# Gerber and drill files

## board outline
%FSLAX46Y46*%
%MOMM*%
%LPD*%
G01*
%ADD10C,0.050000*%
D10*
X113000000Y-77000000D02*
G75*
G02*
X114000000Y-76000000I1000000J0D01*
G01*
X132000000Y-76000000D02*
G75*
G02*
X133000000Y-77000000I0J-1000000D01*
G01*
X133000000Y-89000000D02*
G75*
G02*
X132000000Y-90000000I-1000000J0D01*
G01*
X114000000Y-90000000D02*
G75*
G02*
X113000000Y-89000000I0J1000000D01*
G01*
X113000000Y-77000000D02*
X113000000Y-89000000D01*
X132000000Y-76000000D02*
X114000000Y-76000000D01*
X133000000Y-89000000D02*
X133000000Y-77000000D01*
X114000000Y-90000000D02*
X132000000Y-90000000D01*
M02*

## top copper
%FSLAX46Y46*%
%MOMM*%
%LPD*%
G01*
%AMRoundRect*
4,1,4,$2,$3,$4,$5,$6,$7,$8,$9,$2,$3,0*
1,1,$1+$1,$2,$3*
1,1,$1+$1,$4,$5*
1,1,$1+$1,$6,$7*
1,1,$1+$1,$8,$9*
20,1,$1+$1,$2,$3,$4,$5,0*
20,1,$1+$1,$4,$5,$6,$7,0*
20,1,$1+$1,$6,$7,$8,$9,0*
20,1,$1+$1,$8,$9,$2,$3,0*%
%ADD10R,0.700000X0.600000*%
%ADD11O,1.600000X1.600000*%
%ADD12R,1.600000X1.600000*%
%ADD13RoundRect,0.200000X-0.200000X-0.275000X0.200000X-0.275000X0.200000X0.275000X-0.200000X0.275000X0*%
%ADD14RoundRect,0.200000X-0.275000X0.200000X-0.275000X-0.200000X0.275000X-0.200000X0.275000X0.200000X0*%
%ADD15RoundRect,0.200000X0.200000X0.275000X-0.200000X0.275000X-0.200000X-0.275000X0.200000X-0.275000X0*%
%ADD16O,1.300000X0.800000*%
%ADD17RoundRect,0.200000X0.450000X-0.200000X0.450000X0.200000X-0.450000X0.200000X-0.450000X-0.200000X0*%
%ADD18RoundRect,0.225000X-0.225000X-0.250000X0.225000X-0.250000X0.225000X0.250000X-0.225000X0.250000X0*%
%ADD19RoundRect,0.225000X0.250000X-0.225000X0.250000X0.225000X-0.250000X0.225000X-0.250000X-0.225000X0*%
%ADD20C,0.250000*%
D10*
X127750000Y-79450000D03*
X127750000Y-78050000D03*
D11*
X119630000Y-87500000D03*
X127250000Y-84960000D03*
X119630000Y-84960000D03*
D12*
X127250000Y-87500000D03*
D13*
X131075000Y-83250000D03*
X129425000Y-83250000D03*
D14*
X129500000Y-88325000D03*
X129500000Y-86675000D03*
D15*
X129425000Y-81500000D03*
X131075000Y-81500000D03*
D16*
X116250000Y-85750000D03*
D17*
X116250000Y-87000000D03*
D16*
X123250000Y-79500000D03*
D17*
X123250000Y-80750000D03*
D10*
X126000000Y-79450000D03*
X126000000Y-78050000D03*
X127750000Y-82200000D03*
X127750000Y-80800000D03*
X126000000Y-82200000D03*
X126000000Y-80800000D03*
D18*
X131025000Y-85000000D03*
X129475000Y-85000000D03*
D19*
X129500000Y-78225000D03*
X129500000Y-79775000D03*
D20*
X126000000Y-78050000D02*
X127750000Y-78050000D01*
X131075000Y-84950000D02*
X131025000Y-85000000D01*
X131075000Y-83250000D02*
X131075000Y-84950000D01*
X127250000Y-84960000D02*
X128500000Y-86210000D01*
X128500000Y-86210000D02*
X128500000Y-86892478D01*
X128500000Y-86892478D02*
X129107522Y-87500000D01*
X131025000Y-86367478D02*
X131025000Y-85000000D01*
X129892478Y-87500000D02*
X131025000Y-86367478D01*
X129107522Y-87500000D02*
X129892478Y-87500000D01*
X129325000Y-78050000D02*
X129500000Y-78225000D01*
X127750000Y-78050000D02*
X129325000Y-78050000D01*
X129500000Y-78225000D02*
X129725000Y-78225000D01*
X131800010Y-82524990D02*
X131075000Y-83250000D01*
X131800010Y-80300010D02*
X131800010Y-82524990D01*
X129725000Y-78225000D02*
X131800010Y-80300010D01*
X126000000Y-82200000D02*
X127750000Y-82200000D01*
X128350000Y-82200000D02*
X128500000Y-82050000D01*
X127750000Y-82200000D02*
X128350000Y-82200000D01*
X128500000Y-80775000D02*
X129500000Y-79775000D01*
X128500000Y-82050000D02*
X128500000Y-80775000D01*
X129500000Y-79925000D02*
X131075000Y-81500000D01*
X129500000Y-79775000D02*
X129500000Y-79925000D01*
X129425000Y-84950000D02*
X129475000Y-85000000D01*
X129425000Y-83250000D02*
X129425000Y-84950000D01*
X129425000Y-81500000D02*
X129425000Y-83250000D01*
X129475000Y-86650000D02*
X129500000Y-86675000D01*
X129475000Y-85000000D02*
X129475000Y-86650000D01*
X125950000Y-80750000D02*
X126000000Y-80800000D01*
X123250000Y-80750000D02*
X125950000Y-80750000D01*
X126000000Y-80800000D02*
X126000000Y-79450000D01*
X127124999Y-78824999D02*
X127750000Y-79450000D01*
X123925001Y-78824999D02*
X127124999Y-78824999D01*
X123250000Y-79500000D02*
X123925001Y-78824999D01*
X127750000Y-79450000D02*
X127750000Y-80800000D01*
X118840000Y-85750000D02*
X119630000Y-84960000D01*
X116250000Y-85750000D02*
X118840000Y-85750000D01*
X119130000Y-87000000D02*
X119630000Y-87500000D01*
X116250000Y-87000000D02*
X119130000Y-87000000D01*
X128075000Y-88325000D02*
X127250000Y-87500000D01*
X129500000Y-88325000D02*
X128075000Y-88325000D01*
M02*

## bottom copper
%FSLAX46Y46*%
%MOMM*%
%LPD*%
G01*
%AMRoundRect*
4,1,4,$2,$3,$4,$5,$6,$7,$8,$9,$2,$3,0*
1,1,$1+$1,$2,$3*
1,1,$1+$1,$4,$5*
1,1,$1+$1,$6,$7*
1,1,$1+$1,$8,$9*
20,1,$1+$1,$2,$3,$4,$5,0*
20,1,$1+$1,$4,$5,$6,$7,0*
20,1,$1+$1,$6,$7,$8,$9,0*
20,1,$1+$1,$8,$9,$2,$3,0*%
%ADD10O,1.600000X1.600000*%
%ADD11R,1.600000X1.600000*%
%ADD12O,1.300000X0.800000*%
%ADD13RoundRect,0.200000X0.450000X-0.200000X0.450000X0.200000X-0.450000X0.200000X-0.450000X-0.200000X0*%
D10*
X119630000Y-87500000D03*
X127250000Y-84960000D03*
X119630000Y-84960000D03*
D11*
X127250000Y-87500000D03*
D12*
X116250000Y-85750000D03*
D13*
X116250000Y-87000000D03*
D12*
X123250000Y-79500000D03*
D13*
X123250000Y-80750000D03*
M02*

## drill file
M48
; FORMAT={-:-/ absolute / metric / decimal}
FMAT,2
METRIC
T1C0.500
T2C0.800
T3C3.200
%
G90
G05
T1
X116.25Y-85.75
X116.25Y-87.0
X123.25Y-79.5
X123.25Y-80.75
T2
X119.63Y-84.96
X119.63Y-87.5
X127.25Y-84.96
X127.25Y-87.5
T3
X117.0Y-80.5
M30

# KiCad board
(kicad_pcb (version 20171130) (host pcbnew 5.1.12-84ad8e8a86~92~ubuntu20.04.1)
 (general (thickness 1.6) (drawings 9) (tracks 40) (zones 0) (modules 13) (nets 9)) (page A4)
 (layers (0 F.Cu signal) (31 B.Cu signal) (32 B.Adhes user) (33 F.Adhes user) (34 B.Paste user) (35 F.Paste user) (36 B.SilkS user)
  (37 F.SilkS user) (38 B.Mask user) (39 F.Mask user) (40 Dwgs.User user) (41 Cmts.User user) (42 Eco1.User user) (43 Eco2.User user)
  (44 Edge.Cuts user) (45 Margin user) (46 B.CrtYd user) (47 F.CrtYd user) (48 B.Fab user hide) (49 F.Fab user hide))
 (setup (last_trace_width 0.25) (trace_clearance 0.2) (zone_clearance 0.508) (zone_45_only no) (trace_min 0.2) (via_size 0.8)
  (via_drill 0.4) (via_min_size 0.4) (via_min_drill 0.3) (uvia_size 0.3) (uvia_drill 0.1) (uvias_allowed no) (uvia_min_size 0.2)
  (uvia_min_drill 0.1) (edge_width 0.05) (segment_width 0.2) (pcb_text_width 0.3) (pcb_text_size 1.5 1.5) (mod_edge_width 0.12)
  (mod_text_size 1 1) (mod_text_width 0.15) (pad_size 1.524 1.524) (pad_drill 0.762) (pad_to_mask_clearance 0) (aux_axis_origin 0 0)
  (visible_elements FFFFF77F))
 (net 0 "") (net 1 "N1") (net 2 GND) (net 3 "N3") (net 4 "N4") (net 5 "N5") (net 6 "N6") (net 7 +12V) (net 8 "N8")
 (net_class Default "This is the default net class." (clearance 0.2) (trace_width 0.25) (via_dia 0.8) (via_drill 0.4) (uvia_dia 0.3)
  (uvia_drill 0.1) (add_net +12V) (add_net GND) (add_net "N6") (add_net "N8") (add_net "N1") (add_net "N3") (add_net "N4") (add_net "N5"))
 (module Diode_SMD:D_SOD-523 (layer F.Cu) (at 127.75 78.75 90)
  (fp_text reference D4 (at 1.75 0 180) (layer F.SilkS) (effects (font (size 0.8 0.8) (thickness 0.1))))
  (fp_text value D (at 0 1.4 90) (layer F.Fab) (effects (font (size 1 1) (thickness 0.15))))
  (pad 1 smd rect (at -0.7 0 270) (size 0.6 0.7) (layers F.Cu F.Paste F.Mask) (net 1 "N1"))
  (pad 2 smd rect (at 0.7 0 270) (size 0.6 0.7) (layers F.Cu F.Paste F.Mask) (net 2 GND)))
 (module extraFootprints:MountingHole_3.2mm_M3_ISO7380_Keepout (layer F.Cu) (at 117 80.5)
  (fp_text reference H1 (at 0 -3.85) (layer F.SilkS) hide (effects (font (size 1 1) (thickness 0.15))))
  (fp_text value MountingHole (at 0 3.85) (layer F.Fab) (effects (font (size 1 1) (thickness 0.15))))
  (pad "" np_thru_hole circle (at 0 0) (size 3.2 3.2) (drill 3.2) (layers *.Cu *.Mask) (solder_mask_margin 1.45) (clearance 1.45)))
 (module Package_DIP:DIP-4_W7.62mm (layer F.Cu) (at 127.25 87.5 180)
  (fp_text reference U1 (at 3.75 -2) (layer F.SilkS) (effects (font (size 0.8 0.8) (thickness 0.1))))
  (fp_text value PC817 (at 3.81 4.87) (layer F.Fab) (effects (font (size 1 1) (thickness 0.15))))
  (pad 4 thru_hole oval (at 7.62 0 180) (size 1.6 1.6) (drill 0.8) (layers *.Cu *.Mask) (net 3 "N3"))
  (pad 2 thru_hole oval (at 0 2.54 180) (size 1.6 1.6) (drill 0.8) (layers *.Cu *.Mask) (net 2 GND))
  (pad 3 thru_hole oval (at 7.62 2.54 180) (size 1.6 1.6) (drill 0.8) (layers *.Cu *.Mask) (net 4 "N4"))
  (pad 1 thru_hole rect (at 0 0 180) (size 1.6 1.6) (drill 0.8) (layers *.Cu *.Mask) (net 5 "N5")))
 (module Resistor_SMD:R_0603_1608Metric (layer F.Cu) (at 130.25 83.25)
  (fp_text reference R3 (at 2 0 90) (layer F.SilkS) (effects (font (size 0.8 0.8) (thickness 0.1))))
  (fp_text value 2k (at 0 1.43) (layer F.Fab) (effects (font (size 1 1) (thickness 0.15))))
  (pad 2 smd roundrect (at 0.825 0) (size 0.8 0.95) (layers F.Cu F.Paste F.Mask) (roundrect_rratio 0.25) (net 2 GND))
  (pad 1 smd roundrect (at -0.825 0) (size 0.8 0.95) (layers F.Cu F.Paste F.Mask) (roundrect_rratio 0.25) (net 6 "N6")))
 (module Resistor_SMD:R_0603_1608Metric (layer F.Cu) (at 129.5 87.5 270)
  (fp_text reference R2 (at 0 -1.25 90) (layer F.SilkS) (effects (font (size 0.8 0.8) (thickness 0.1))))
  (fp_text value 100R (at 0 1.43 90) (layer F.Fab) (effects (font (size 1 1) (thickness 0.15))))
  (pad 2 smd roundrect (at 0.825 0 270) (size 0.8 0.95) (layers F.Cu F.Paste F.Mask) (roundrect_rratio 0.25) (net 5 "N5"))
  (pad 1 smd roundrect (at -0.825 0 270) (size 0.8 0.95) (layers F.Cu F.Paste F.Mask) (roundrect_rratio 0.25) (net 6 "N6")))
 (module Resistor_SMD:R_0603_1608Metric (layer F.Cu) (at 130.25 81.5 180)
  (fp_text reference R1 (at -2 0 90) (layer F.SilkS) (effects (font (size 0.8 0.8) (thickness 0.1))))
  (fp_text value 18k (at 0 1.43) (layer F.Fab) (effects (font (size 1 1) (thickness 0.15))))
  (pad 2 smd roundrect (at 0.825 0 180) (size 0.8 0.95) (layers F.Cu F.Paste F.Mask) (roundrect_rratio 0.25) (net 6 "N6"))
  (pad 1 smd roundrect (at -0.825 0 180) (size 0.8 0.95) (layers F.Cu F.Paste F.Mask) (roundrect_rratio 0.25) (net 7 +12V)))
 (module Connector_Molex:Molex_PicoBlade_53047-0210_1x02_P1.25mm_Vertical (layer F.Cu) (at 116.25 87 90)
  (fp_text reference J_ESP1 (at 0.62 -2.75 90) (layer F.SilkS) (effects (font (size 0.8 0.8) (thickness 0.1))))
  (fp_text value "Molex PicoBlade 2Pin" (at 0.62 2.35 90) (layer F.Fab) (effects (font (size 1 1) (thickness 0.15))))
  (pad 2 thru_hole oval (at 1.25 0 90) (size 0.8 1.3) (drill 0.5) (layers *.Cu *.Mask) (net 4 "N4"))
  (pad 1 thru_hole roundrect (at 0 0 90) (size 0.8 1.3) (drill 0.5) (layers *.Cu *.Mask) (roundrect_rratio 0.25) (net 3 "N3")))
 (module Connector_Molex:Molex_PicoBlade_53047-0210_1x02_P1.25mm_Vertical (layer F.Cu) (at 123.25 80.75 90)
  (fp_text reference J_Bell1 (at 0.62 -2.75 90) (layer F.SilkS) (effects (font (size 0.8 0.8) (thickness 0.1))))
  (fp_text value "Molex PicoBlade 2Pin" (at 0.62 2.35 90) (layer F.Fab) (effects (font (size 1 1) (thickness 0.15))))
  (pad 2 thru_hole oval (at 1.25 0 90) (size 0.8 1.3) (drill 0.5) (layers *.Cu *.Mask) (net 1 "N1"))
  (pad 1 thru_hole roundrect (at 0 0 90) (size 0.8 1.3) (drill 0.5) (layers *.Cu *.Mask) (roundrect_rratio 0.25) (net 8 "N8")))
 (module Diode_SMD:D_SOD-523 (layer F.Cu) (at 126 78.75 90)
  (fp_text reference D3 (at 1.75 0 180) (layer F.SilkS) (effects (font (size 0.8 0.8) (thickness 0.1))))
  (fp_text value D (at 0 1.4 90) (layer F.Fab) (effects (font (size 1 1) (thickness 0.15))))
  (pad 1 smd rect (at -0.7 0 270) (size 0.6 0.7) (layers F.Cu F.Paste F.Mask) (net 8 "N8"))
  (pad 2 smd rect (at 0.7 0 270) (size 0.6 0.7) (layers F.Cu F.Paste F.Mask) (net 2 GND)))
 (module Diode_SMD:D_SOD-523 (layer F.Cu) (at 127.75 81.5 90)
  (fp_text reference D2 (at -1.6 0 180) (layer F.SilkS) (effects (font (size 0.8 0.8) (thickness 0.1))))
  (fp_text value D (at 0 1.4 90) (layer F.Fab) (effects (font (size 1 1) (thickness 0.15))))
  (pad 1 smd rect (at -0.7 0 270) (size 0.6 0.7) (layers F.Cu F.Paste F.Mask) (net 7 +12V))
  (pad 2 smd rect (at 0.7 0 270) (size 0.6 0.7) (layers F.Cu F.Paste F.Mask) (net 1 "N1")))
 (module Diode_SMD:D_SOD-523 (layer F.Cu) (at 126 81.5 90)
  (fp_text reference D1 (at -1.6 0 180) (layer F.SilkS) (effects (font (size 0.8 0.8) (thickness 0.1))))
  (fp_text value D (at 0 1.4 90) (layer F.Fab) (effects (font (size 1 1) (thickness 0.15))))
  (pad 1 smd rect (at -0.7 0 270) (size 0.6 0.7) (layers F.Cu F.Paste F.Mask) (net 7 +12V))
  (pad 2 smd rect (at 0.7 0 270) (size 0.6 0.7) (layers F.Cu F.Paste F.Mask) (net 8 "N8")))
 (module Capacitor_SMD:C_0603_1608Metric (layer F.Cu) (at 130.25 85)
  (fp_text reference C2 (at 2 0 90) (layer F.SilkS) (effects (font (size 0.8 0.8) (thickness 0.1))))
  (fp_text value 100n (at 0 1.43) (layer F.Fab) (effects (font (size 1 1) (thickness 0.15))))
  (pad 2 smd roundrect (at 0.775 0) (size 0.9 0.95) (layers F.Cu F.Paste F.Mask) (roundrect_rratio 0.25) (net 2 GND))
  (pad 1 smd roundrect (at -0.775 0) (size 0.9 0.95) (layers F.Cu F.Paste F.Mask) (roundrect_rratio 0.25) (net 6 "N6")))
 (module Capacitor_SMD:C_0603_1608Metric (layer F.Cu) (at 129.5 79 90)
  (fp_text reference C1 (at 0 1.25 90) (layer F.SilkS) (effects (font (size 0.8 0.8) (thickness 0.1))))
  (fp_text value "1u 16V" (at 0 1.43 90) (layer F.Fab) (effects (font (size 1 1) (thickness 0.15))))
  (pad 2 smd roundrect (at 0.775 0 90) (size 0.9 0.95) (layers F.Cu F.Paste F.Mask) (roundrect_rratio 0.25) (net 2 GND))
  (pad 1 smd roundrect (at -0.775 0 90) (size 0.9 0.95) (layers F.Cu F.Paste F.Mask) (roundrect_rratio 0.25) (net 7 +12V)))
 (gr_arc (start 114 77) (end 114 76) (angle -90) (layer Edge.Cuts) (width 0.05))
 (gr_arc (start 132 77) (end 133 77) (angle -90) (layer Edge.Cuts) (width 0.05))
 (gr_arc (start 132 89) (end 132 90) (angle -90) (layer Edge.Cuts) (width 0.05))
 (gr_arc (start 114 89) (end 113 89) (angle -90) (layer Edge.Cuts) (width 0.05))
 (gr_line (start 113 77) (end 113 89) (layer Edge.Cuts) (width 0.05))
 (gr_line (start 132 76) (end 114 76) (layer Edge.Cuts) (width 0.05))
 (gr_line (start 133 89) (end 133 77) (layer Edge.Cuts) (width 0.05))
 (gr_line (start 114 90) (end 132 90) (layer Edge.Cuts) (width 0.05))
 (segment (start 126 78.05) (end 127.75 78.05) (width 0.25) (layer F.Cu) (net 2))
 (segment (start 131.075 84.95) (end 131.025 85) (width 0.25) (layer F.Cu) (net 2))
 (segment (start 131.075 83.25) (end 131.075 84.95) (width 0.25) (layer F.Cu) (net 2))
 (segment (start 127.25 84.96) (end 128.5 86.21) (width 0.25) (layer F.Cu) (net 2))
 (segment (start 128.5 86.21) (end 128.5 86.892478) (width 0.25) (layer F.Cu) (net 2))
 (segment (start 128.5 86.892478) (end 129.107522 87.5) (width 0.25) (layer F.Cu) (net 2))
 (segment (start 131.025 86.367478) (end 131.025 85) (width 0.25) (layer F.Cu) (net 2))
 (segment (start 129.892478 87.5) (end 131.025 86.367478) (width 0.25) (layer F.Cu) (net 2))
 (segment (start 129.107522 87.5) (end 129.892478 87.5) (width 0.25) (layer F.Cu) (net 2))
 (segment (start 129.325 78.05) (end 129.5 78.225) (width 0.25) (layer F.Cu) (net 2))
 (segment (start 127.75 78.05) (end 129.325 78.05) (width 0.25) (layer F.Cu) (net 2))
 (segment (start 129.5 78.225) (end 129.725 78.225) (width 0.25) (layer F.Cu) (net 2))
 (segment (start 131.80001 82.52499) (end 131.075 83.25) (width 0.25) (layer F.Cu) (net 2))
 (segment (start 131.80001 80.30001) (end 131.80001 82.52499) (width 0.25) (layer F.Cu) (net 2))
 (segment (start 129.725 78.225) (end 131.80001 80.30001) (width 0.25) (layer F.Cu) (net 2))
 (segment (start 126 82.2) (end 127.75 82.2) (width 0.25) (layer F.Cu) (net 7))
 (segment (start 128.35 82.2) (end 128.5 82.05) (width 0.25) (layer F.Cu) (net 7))
 (segment (start 127.75 82.2) (end 128.35 82.2) (width 0.25) (layer F.Cu) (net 7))
 (segment (start 128.5 80.775) (end 129.5 79.775) (width 0.25) (layer F.Cu) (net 7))
 (segment (start 128.5 82.05) (end 128.5 80.775) (width 0.25) (layer F.Cu) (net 7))
 (segment (start 129.5 79.925) (end 131.075 81.5) (width 0.25) (layer F.Cu) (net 7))
 (segment (start 129.5 79.775) (end 129.5 79.925) (width 0.25) (layer F.Cu) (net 7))
 (segment (start 129.425 84.95) (end 129.475 85) (width 0.25) (layer F.Cu) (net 6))
 (segment (start 129.425 83.25) (end 129.425 84.95) (width 0.25) (layer F.Cu) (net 6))
 (segment (start 129.425 81.5) (end 129.425 83.25) (width 0.25) (layer F.Cu) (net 6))
 (segment (start 129.475 86.65) (end 129.5 86.675) (width 0.25) (layer F.Cu) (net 6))
 (segment (start 129.475 85) (end 129.475 86.65) (width 0.25) (layer F.Cu) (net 6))
 (segment (start 125.95 80.75) (end 126 80.8) (width 0.25) (layer F.Cu) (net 8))
 (segment (start 123.25 80.75) (end 125.95 80.75) (width 0.25) (layer F.Cu) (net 8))
 (segment (start 126 80.8) (end 126 79.45) (width 0.25) (layer F.Cu) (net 8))
 (segment (start 127.124999 78.824999) (end 127.75 79.45) (width 0.25) (layer F.Cu) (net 1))
 (segment (start 123.925001 78.824999) (end 127.124999 78.824999) (width 0.25) (layer F.Cu) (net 1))
 (segment (start 123.25 79.5) (end 123.925001 78.824999) (width 0.25) (layer F.Cu) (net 1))
 (segment (start 127.75 79.45) (end 127.75 80.8) (width 0.25) (layer F.Cu) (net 1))
 (segment (start 118.84 85.75) (end 119.63 84.96) (width 0.25) (layer F.Cu) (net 4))
 (segment (start 116.25 85.75) (end 118.84 85.75) (width 0.25) (layer F.Cu) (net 4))
 (segment (start 119.13 87) (end 119.63 87.5) (width 0.25) (layer F.Cu) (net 3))
 (segment (start 116.25 87) (end 119.13 87) (width 0.25) (layer F.Cu) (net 3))
 (segment (start 128.075 88.325) (end 127.25 87.5) (width 0.25) (layer F.Cu) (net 5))
 (segment (start 129.5 88.325) (end 128.075 88.325) (width 0.25) (layer F.Cu) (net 5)))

